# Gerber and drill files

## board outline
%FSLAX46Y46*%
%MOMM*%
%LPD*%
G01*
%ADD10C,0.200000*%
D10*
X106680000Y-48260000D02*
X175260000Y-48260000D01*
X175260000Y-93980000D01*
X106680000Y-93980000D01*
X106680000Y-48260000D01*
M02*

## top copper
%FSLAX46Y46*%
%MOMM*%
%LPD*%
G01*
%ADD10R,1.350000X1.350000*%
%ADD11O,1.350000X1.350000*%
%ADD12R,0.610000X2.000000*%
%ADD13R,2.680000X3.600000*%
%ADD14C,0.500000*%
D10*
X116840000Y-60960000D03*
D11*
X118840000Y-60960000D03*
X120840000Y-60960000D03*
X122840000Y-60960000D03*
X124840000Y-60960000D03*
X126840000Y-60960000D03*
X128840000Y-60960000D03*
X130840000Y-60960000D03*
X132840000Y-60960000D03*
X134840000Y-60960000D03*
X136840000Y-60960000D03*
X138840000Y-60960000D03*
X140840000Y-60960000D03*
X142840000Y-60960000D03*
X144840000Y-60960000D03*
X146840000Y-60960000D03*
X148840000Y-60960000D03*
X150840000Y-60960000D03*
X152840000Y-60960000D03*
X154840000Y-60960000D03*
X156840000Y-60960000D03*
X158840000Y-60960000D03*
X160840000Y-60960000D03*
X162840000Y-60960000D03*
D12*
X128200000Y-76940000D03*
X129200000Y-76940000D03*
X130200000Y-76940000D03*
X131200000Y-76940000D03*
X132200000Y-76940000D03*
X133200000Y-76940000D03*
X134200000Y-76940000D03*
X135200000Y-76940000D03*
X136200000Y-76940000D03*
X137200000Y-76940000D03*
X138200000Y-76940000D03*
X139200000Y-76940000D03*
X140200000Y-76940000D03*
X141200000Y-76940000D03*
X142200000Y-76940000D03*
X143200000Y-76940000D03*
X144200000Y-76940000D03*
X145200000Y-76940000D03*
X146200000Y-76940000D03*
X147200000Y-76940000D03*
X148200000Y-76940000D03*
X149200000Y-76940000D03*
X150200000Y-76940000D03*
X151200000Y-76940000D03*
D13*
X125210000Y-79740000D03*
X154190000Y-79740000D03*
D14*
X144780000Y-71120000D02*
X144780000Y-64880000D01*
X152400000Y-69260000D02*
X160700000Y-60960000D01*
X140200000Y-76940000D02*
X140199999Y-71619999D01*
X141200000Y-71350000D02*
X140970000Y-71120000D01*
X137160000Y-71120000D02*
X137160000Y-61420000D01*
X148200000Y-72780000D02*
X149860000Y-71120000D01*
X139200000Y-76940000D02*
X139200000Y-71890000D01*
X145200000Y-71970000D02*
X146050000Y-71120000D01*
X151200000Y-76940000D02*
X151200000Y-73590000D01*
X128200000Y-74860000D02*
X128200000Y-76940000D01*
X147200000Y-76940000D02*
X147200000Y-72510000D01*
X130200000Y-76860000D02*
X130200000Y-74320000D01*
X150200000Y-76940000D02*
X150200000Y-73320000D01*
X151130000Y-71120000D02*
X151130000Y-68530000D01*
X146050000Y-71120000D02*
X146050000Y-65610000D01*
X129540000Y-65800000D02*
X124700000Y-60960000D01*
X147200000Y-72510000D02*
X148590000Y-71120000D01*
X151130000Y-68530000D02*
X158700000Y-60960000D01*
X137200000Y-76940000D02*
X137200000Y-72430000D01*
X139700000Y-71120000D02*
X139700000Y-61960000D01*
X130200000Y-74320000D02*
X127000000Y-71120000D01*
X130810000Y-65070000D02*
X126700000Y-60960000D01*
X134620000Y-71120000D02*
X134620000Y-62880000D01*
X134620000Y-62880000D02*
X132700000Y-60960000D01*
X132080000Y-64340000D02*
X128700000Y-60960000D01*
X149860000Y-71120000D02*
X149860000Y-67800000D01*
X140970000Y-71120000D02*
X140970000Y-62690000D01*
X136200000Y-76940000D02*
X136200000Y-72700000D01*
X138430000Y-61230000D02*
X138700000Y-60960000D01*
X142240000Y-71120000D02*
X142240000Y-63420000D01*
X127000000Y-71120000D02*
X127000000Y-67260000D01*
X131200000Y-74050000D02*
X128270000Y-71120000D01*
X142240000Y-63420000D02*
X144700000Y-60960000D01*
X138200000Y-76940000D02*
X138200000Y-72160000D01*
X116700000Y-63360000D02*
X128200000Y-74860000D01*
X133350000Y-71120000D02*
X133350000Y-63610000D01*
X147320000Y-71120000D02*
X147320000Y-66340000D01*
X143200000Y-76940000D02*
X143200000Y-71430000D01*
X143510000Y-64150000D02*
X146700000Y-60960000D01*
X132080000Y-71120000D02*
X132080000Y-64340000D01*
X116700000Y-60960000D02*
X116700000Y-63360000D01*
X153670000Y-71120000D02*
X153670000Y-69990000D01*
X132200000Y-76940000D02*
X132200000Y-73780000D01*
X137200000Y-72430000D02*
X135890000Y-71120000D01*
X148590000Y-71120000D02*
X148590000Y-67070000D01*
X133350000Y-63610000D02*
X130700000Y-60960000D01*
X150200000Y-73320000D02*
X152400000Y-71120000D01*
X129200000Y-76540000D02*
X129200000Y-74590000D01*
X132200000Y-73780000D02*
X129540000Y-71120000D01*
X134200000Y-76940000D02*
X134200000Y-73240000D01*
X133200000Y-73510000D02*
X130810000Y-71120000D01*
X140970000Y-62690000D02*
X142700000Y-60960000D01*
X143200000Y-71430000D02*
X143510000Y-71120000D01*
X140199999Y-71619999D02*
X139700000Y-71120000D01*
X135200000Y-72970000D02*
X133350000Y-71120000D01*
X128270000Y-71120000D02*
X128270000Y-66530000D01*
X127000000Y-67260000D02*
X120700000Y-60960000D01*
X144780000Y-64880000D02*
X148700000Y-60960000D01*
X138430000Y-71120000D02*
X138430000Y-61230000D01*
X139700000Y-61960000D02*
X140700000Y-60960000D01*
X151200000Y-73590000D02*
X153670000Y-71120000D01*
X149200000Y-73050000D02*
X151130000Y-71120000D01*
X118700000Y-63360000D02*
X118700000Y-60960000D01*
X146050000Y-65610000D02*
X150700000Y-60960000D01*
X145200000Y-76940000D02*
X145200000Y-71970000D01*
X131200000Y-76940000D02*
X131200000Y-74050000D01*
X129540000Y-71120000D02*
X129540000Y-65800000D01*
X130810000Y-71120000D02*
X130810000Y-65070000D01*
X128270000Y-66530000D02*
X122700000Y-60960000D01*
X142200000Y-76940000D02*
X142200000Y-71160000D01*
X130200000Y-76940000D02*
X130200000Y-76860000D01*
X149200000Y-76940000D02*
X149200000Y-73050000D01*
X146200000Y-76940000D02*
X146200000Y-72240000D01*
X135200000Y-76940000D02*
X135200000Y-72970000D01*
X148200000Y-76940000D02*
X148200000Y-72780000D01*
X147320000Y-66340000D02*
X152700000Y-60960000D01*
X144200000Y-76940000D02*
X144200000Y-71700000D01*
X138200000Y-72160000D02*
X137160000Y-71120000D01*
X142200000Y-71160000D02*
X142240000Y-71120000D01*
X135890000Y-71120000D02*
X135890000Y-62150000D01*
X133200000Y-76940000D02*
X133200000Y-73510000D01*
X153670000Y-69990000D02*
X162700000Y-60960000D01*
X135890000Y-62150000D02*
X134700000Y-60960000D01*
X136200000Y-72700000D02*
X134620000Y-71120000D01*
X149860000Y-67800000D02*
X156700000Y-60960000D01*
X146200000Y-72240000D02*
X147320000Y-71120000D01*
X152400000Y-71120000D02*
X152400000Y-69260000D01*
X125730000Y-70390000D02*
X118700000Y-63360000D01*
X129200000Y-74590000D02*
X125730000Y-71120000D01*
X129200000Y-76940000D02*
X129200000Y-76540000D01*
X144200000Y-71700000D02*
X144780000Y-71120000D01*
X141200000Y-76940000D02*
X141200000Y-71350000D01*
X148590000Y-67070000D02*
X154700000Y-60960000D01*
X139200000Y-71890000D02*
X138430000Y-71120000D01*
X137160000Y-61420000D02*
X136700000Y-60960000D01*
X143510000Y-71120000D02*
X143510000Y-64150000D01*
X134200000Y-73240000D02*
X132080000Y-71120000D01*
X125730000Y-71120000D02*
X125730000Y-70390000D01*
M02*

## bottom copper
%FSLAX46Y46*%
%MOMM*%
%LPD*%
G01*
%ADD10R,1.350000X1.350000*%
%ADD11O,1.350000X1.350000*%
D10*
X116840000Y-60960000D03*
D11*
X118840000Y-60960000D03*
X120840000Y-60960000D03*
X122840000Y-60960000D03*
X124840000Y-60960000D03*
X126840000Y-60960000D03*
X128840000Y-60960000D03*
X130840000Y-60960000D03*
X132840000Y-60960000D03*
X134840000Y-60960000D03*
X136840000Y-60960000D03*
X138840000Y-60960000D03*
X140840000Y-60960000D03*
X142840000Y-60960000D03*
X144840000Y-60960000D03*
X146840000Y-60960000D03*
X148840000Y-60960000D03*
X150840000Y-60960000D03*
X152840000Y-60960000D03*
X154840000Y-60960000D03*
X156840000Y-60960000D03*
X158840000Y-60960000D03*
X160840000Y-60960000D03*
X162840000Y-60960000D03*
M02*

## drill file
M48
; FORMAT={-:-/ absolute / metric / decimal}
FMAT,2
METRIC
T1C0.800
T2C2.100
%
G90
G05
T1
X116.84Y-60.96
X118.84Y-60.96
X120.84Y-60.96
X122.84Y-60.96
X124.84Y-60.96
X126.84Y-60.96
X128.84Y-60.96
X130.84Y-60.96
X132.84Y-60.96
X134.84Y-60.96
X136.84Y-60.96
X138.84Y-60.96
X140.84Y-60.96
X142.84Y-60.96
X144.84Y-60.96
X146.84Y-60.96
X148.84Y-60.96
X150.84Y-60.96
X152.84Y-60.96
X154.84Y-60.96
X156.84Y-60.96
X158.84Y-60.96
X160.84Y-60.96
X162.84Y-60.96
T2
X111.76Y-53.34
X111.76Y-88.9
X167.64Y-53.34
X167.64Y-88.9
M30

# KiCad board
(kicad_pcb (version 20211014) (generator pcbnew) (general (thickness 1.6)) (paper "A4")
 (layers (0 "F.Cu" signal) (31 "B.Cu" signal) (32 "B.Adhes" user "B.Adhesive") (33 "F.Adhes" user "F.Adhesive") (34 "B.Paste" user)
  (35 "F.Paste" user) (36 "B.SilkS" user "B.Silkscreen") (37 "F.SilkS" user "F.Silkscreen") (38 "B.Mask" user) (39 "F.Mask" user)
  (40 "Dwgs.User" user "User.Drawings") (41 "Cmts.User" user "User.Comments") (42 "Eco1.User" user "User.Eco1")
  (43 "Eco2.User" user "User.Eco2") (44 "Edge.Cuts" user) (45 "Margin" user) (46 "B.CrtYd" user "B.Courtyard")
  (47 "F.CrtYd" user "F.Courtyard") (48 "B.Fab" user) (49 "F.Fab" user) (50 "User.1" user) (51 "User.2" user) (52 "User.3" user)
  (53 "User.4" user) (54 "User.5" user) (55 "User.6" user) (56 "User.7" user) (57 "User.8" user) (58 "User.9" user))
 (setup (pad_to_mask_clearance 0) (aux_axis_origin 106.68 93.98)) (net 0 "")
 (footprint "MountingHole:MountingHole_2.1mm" (layer "F.Cu") (at 111.76 53.34)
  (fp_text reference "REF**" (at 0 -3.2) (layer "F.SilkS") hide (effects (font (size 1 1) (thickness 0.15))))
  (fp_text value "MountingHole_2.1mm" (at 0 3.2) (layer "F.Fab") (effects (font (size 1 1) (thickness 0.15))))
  (pad "" np_thru_hole circle (at 0 0) (size 2.1 2.1) (drill 2.1) (layers *.Cu *.Mask)))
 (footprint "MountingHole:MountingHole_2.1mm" (layer "F.Cu") (at 167.64 53.34)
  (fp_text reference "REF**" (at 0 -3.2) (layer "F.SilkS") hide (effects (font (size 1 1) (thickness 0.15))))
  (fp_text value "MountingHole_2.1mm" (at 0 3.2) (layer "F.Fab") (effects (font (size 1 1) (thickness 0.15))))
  (pad "" np_thru_hole circle (at 0 0) (size 2.1 2.1) (drill 2.1) (layers *.Cu *.Mask)))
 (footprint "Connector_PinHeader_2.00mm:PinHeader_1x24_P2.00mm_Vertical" (layer "F.Cu") (at 116.84 60.96 90)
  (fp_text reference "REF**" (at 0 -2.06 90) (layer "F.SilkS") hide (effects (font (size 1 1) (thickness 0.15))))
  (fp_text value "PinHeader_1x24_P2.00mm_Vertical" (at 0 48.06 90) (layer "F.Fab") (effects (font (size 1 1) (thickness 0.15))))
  (pad "1" thru_hole rect (at 0 0 90) (size 1.35 1.35) (drill 0.8) (layers *.Cu *.Mask))
  (pad "2" thru_hole oval (at 0 2 90) (size 1.35 1.35) (drill 0.8) (layers *.Cu *.Mask))
  (pad "3" thru_hole oval (at 0 4 90) (size 1.35 1.35) (drill 0.8) (layers *.Cu *.Mask))
  (pad "4" thru_hole oval (at 0 6 90) (size 1.35 1.35) (drill 0.8) (layers *.Cu *.Mask))
  (pad "5" thru_hole oval (at 0 8 90) (size 1.35 1.35) (drill 0.8) (layers *.Cu *.Mask))
  (pad "6" thru_hole oval (at 0 10 90) (size 1.35 1.35) (drill 0.8) (layers *.Cu *.Mask))
  (pad "7" thru_hole oval (at 0 12 90) (size 1.35 1.35) (drill 0.8) (layers *.Cu *.Mask))
  (pad "8" thru_hole oval (at 0 14 90) (size 1.35 1.35) (drill 0.8) (layers *.Cu *.Mask))
  (pad "9" thru_hole oval (at 0 16 90) (size 1.35 1.35) (drill 0.8) (layers *.Cu *.Mask))
  (pad "10" thru_hole oval (at 0 18 90) (size 1.35 1.35) (drill 0.8) (layers *.Cu *.Mask))
  (pad "11" thru_hole oval (at 0 20 90) (size 1.35 1.35) (drill 0.8) (layers *.Cu *.Mask))
  (pad "12" thru_hole oval (at 0 22 90) (size 1.35 1.35) (drill 0.8) (layers *.Cu *.Mask))
  (pad "13" thru_hole oval (at 0 24 90) (size 1.35 1.35) (drill 0.8) (layers *.Cu *.Mask))
  (pad "14" thru_hole oval (at 0 26 90) (size 1.35 1.35) (drill 0.8) (layers *.Cu *.Mask))
  (pad "15" thru_hole oval (at 0 28 90) (size 1.35 1.35) (drill 0.8) (layers *.Cu *.Mask))
  (pad "16" thru_hole oval (at 0 30 90) (size 1.35 1.35) (drill 0.8) (layers *.Cu *.Mask))
  (pad "17" thru_hole oval (at 0 32 90) (size 1.35 1.35) (drill 0.8) (layers *.Cu *.Mask))
  (pad "18" thru_hole oval (at 0 34 90) (size 1.35 1.35) (drill 0.8) (layers *.Cu *.Mask))
  (pad "19" thru_hole oval (at 0 36 90) (size 1.35 1.35) (drill 0.8) (layers *.Cu *.Mask))
  (pad "20" thru_hole oval (at 0 38 90) (size 1.35 1.35) (drill 0.8) (layers *.Cu *.Mask))
  (pad "21" thru_hole oval (at 0 40 90) (size 1.35 1.35) (drill 0.8) (layers *.Cu *.Mask))
  (pad "22" thru_hole oval (at 0 42 90) (size 1.35 1.35) (drill 0.8) (layers *.Cu *.Mask))
  (pad "23" thru_hole oval (at 0 44 90) (size 1.35 1.35) (drill 0.8) (layers *.Cu *.Mask))
  (pad "24" thru_hole oval (at 0 46 90) (size 1.35 1.35) (drill 0.8) (layers *.Cu *.Mask)))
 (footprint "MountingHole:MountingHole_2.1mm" (layer "F.Cu") (at 111.76 88.9)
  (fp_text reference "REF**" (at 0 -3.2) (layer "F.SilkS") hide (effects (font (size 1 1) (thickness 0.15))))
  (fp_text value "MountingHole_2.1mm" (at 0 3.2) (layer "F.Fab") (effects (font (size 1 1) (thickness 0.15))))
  (pad "" np_thru_hole circle (at 0 0) (size 2.1 2.1) (drill 2.1) (layers *.Cu *.Mask)))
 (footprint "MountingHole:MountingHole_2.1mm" (layer "F.Cu") (at 167.64 88.9)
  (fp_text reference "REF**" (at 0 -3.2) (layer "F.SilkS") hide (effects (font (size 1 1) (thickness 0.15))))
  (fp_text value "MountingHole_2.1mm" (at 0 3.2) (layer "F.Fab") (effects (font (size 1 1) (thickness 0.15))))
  (pad "" np_thru_hole circle (at 0 0) (size 2.1 2.1) (drill 2.1) (layers *.Cu *.Mask)))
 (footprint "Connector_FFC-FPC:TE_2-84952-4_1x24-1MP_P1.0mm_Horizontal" (layer "F.Cu") (at 139.7 78.74)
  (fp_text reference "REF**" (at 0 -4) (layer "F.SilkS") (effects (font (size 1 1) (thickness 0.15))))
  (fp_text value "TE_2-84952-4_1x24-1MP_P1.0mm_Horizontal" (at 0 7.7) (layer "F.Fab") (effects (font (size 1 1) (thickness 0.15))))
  (pad "1" smd rect (at -11.5 -1.8) (size 0.61 2) (layers "F.Cu" "F.Paste" "F.Mask"))
  (pad "2" smd rect (at -10.5 -1.8) (size 0.61 2) (layers "F.Cu" "F.Paste" "F.Mask"))
  (pad "3" smd rect (at -9.5 -1.8) (size 0.61 2) (layers "F.Cu" "F.Paste" "F.Mask"))
  (pad "4" smd rect (at -8.5 -1.8) (size 0.61 2) (layers "F.Cu" "F.Paste" "F.Mask"))
  (pad "5" smd rect (at -7.5 -1.8) (size 0.61 2) (layers "F.Cu" "F.Paste" "F.Mask"))
  (pad "6" smd rect (at -6.5 -1.8) (size 0.61 2) (layers "F.Cu" "F.Paste" "F.Mask"))
  (pad "7" smd rect (at -5.5 -1.8) (size 0.61 2) (layers "F.Cu" "F.Paste" "F.Mask"))
  (pad "8" smd rect (at -4.5 -1.8) (size 0.61 2) (layers "F.Cu" "F.Paste" "F.Mask"))
  (pad "9" smd rect (at -3.5 -1.8) (size 0.61 2) (layers "F.Cu" "F.Paste" "F.Mask"))
  (pad "10" smd rect (at -2.5 -1.8) (size 0.61 2) (layers "F.Cu" "F.Paste" "F.Mask"))
  (pad "11" smd rect (at -1.5 -1.8) (size 0.61 2) (layers "F.Cu" "F.Paste" "F.Mask"))
  (pad "12" smd rect (at -0.5 -1.8) (size 0.61 2) (layers "F.Cu" "F.Paste" "F.Mask"))
  (pad "13" smd rect (at 0.5 -1.8) (size 0.61 2) (layers "F.Cu" "F.Paste" "F.Mask"))
  (pad "14" smd rect (at 1.5 -1.8) (size 0.61 2) (layers "F.Cu" "F.Paste" "F.Mask"))
  (pad "15" smd rect (at 2.5 -1.8) (size 0.61 2) (layers "F.Cu" "F.Paste" "F.Mask"))
  (pad "16" smd rect (at 3.5 -1.8) (size 0.61 2) (layers "F.Cu" "F.Paste" "F.Mask"))
  (pad "17" smd rect (at 4.5 -1.8) (size 0.61 2) (layers "F.Cu" "F.Paste" "F.Mask"))
  (pad "18" smd rect (at 5.5 -1.8) (size 0.61 2) (layers "F.Cu" "F.Paste" "F.Mask"))
  (pad "19" smd rect (at 6.5 -1.8) (size 0.61 2) (layers "F.Cu" "F.Paste" "F.Mask"))
  (pad "20" smd rect (at 7.5 -1.8) (size 0.61 2) (layers "F.Cu" "F.Paste" "F.Mask"))
  (pad "21" smd rect (at 8.5 -1.8) (size 0.61 2) (layers "F.Cu" "F.Paste" "F.Mask"))
  (pad "22" smd rect (at 9.5 -1.8) (size 0.61 2) (layers "F.Cu" "F.Paste" "F.Mask"))
  (pad "23" smd rect (at 10.5 -1.8) (size 0.61 2) (layers "F.Cu" "F.Paste" "F.Mask"))
  (pad "24" smd rect (at 11.5 -1.8) (size 0.61 2) (layers "F.Cu" "F.Paste" "F.Mask"))
  (pad "MP" smd rect (at -14.49 1) (size 2.68 3.6) (layers "F.Cu" "F.Paste" "F.Mask"))
  (pad "MP" smd rect (at 14.49 1) (size 2.68 3.6) (layers "F.Cu" "F.Paste" "F.Mask")))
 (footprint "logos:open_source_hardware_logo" (layer "F.Cu") (at 167.64 71.12)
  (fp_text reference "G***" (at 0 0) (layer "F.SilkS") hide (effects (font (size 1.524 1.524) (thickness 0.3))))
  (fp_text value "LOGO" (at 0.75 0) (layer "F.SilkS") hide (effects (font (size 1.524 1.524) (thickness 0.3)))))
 (gr_rect (start 175.26 48.26) (end 106.68 93.98) (layer "Edge.Cuts") (width 0.2) (fill none))
 (segment (start 144.78 71.12) (end 144.78 64.88) (width 0.5) (layer "F.Cu") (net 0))
 (segment (start 152.4 69.26) (end 160.7 60.96) (width 0.5) (layer "F.Cu") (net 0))
 (segment (start 140.2 76.94) (end 140.199999 71.619999) (width 0.5) (layer "F.Cu") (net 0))
 (segment (start 141.2 71.35) (end 140.97 71.12) (width 0.5) (layer "F.Cu") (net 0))
 (segment (start 137.16 71.12) (end 137.16 61.42) (width 0.5) (layer "F.Cu") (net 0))
 (segment (start 148.2 72.78) (end 149.86 71.12) (width 0.5) (layer "F.Cu") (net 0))
 (segment (start 139.2 76.94) (end 139.2 71.89) (width 0.5) (layer "F.Cu") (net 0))
 (segment (start 145.2 71.97) (end 146.05 71.12) (width 0.5) (layer "F.Cu") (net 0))
 (segment (start 151.2 76.94) (end 151.2 73.59) (width 0.5) (layer "F.Cu") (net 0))
 (segment (start 128.2 74.86) (end 128.2 76.94) (width 0.5) (layer "F.Cu") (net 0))
 (segment (start 147.2 76.94) (end 147.2 72.51) (width 0.5) (layer "F.Cu") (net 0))
 (segment (start 130.2 76.86) (end 130.2 74.32) (width 0.5) (layer "F.Cu") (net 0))
 (segment (start 150.2 76.94) (end 150.2 73.32) (width 0.5) (layer "F.Cu") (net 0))
 (segment (start 151.13 71.12) (end 151.13 68.53) (width 0.5) (layer "F.Cu") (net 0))
 (segment (start 146.05 71.12) (end 146.05 65.61) (width 0.5) (layer "F.Cu") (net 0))
 (segment (start 129.54 65.8) (end 124.7 60.96) (width 0.5) (layer "F.Cu") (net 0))
 (segment (start 147.2 72.51) (end 148.59 71.12) (width 0.5) (layer "F.Cu") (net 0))
 (segment (start 151.13 68.53) (end 158.7 60.96) (width 0.5) (layer "F.Cu") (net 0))
 (segment (start 137.2 76.94) (end 137.2 72.43) (width 0.5) (layer "F.Cu") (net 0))
 (segment (start 139.7 71.12) (end 139.7 61.96) (width 0.5) (layer "F.Cu") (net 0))
 (segment (start 130.2 74.32) (end 127 71.12) (width 0.5) (layer "F.Cu") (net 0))
 (segment (start 130.81 65.07) (end 126.7 60.96) (width 0.5) (layer "F.Cu") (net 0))
 (segment (start 134.62 71.12) (end 134.62 62.88) (width 0.5) (layer "F.Cu") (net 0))
 (segment (start 134.62 62.88) (end 132.7 60.96) (width 0.5) (layer "F.Cu") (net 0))
 (segment (start 132.08 64.34) (end 128.7 60.96) (width 0.5) (layer "F.Cu") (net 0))
 (segment (start 149.86 71.12) (end 149.86 67.8) (width 0.5) (layer "F.Cu") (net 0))
 (segment (start 140.97 71.12) (end 140.97 62.69) (width 0.5) (layer "F.Cu") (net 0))
 (segment (start 136.2 76.94) (end 136.2 72.7) (width 0.5) (layer "F.Cu") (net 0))
 (segment (start 138.43 61.23) (end 138.7 60.96) (width 0.5) (layer "F.Cu") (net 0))
 (segment (start 142.24 71.12) (end 142.24 63.42) (width 0.5) (layer "F.Cu") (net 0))
 (segment (start 127 71.12) (end 127 67.26) (width 0.5) (layer "F.Cu") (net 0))
 (segment (start 131.2 74.05) (end 128.27 71.12) (width 0.5) (layer "F.Cu") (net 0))
 (segment (start 142.24 63.42) (end 144.7 60.96) (width 0.5) (layer "F.Cu") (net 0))
 (segment (start 138.2 76.94) (end 138.2 72.16) (width 0.5) (layer "F.Cu") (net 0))
 (segment (start 116.7 63.36) (end 128.2 74.86) (width 0.5) (layer "F.Cu") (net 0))
 (segment (start 133.35 71.12) (end 133.35 63.61) (width 0.5) (layer "F.Cu") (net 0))
 (segment (start 147.32 71.12) (end 147.32 66.34) (width 0.5) (layer "F.Cu") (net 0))
 (segment (start 143.2 76.94) (end 143.2 71.43) (width 0.5) (layer "F.Cu") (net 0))
 (segment (start 143.51 64.15) (end 146.7 60.96) (width 0.5) (layer "F.Cu") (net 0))
 (segment (start 132.08 71.12) (end 132.08 64.34) (width 0.5) (layer "F.Cu") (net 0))
 (segment (start 116.7 60.96) (end 116.7 63.36) (width 0.5) (layer "F.Cu") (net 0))
 (segment (start 153.67 71.12) (end 153.67 69.99) (width 0.5) (layer "F.Cu") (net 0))
 (segment (start 132.2 76.94) (end 132.2 73.78) (width 0.5) (layer "F.Cu") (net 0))
 (segment (start 137.2 72.43) (end 135.89 71.12) (width 0.5) (layer "F.Cu") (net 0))
 (segment (start 148.59 71.12) (end 148.59 67.07) (width 0.5) (layer "F.Cu") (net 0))
 (segment (start 133.35 63.61) (end 130.7 60.96) (width 0.5) (layer "F.Cu") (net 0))
 (segment (start 150.2 73.32) (end 152.4 71.12) (width 0.5) (layer "F.Cu") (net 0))
 (segment (start 129.2 76.54) (end 129.2 74.59) (width 0.5) (layer "F.Cu") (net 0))
 (segment (start 132.2 73.78) (end 129.54 71.12) (width 0.5) (layer "F.Cu") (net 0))
 (segment (start 134.2 76.94) (end 134.2 73.24) (width 0.5) (layer "F.Cu") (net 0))
 (segment (start 133.2 73.51) (end 130.81 71.12) (width 0.5) (layer "F.Cu") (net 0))
 (segment (start 140.97 62.69) (end 142.7 60.96) (width 0.5) (layer "F.Cu") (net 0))
 (segment (start 143.2 71.43) (end 143.51 71.12) (width 0.5) (layer "F.Cu") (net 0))
 (segment (start 140.199999 71.619999) (end 139.7 71.12) (width 0.5) (layer "F.Cu") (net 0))
 (segment (start 135.2 72.97) (end 133.35 71.12) (width 0.5) (layer "F.Cu") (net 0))
 (segment (start 128.27 71.12) (end 128.27 66.53) (width 0.5) (layer "F.Cu") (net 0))
 (segment (start 127 67.26) (end 120.7 60.96) (width 0.5) (layer "F.Cu") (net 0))
 (segment (start 144.78 64.88) (end 148.7 60.96) (width 0.5) (layer "F.Cu") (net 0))
 (segment (start 138.43 71.12) (end 138.43 61.23) (width 0.5) (layer "F.Cu") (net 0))
 (segment (start 139.7 61.96) (end 140.7 60.96) (width 0.5) (layer "F.Cu") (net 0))
 (segment (start 151.2 73.59) (end 153.67 71.12) (width 0.5) (layer "F.Cu") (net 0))
 (segment (start 149.2 73.05) (end 151.13 71.12) (width 0.5) (layer "F.Cu") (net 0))
 (segment (start 118.7 63.36) (end 118.7 60.96) (width 0.5) (layer "F.Cu") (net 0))
 (segment (start 146.05 65.61) (end 150.7 60.96) (width 0.5) (layer "F.Cu") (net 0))
 (segment (start 145.2 76.94) (end 145.2 71.97) (width 0.5) (layer "F.Cu") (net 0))
 (segment (start 131.2 76.94) (end 131.2 74.05) (width 0.5) (layer "F.Cu") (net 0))
 (segment (start 129.54 71.12) (end 129.54 65.8) (width 0.5) (layer "F.Cu") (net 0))
 (segment (start 130.81 71.12) (end 130.81 65.07) (width 0.5) (layer "F.Cu") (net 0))
 (segment (start 128.27 66.53) (end 122.7 60.96) (width 0.5) (layer "F.Cu") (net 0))
 (segment (start 142.2 76.94) (end 142.2 71.16) (width 0.5) (layer "F.Cu") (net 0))
 (segment (start 130.2 76.94) (end 130.2 76.86) (width 0.5) (layer "F.Cu") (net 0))
 (segment (start 149.2 76.94) (end 149.2 73.05) (width 0.5) (layer "F.Cu") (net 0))
 (segment (start 146.2 76.94) (end 146.2 72.24) (width 0.5) (layer "F.Cu") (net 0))
 (segment (start 135.2 76.94) (end 135.2 72.97) (width 0.5) (layer "F.Cu") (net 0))
 (segment (start 148.2 76.94) (end 148.2 72.78) (width 0.5) (layer "F.Cu") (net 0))
 (segment (start 147.32 66.34) (end 152.7 60.96) (width 0.5) (layer "F.Cu") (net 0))
 (segment (start 144.2 76.94) (end 144.2 71.7) (width 0.5) (layer "F.Cu") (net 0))
 (segment (start 138.2 72.16) (end 137.16 71.12) (width 0.5) (layer "F.Cu") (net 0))
 (segment (start 142.2 71.16) (end 142.24 71.12) (width 0.5) (layer "F.Cu") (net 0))
 (segment (start 135.89 71.12) (end 135.89 62.15) (width 0.5) (layer "F.Cu") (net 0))
 (segment (start 133.2 76.94) (end 133.2 73.51) (width 0.5) (layer "F.Cu") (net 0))
 (segment (start 153.67 69.99) (end 162.7 60.96) (width 0.5) (layer "F.Cu") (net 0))
 (segment (start 135.89 62.15) (end 134.7 60.96) (width 0.5) (layer "F.Cu") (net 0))
 (segment (start 136.2 72.7) (end 134.62 71.12) (width 0.5) (layer "F.Cu") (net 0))
 (segment (start 149.86 67.8) (end 156.7 60.96) (width 0.5) (layer "F.Cu") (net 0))
 (segment (start 146.2 72.24) (end 147.32 71.12) (width 0.5) (layer "F.Cu") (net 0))
 (segment (start 152.4 71.12) (end 152.4 69.26) (width 0.5) (layer "F.Cu") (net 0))
 (segment (start 125.73 70.39) (end 118.7 63.36) (width 0.5) (layer "F.Cu") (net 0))
 (segment (start 129.2 74.59) (end 125.73 71.12) (width 0.5) (layer "F.Cu") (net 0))
 (segment (start 129.2 76.94) (end 129.2 76.54) (width 0.5) (layer "F.Cu") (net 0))
 (segment (start 144.2 71.7) (end 144.78 71.12) (width 0.5) (layer "F.Cu") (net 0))
 (segment (start 141.2 76.94) (end 141.2 71.35) (width 0.5) (layer "F.Cu") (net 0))
 (segment (start 148.59 67.07) (end 154.7 60.96) (width 0.5) (layer "F.Cu") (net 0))
 (segment (start 139.2 71.89) (end 138.43 71.12) (width 0.5) (layer "F.Cu") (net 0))
 (segment (start 137.16 61.42) (end 136.7 60.96) (width 0.5) (layer "F.Cu") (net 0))
 (segment (start 143.51 71.12) (end 143.51 64.15) (width 0.5) (layer "F.Cu") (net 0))
 (segment (start 134.2 73.24) (end 132.08 71.12) (width 0.5) (layer "F.Cu") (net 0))
 (segment (start 125.73 71.12) (end 125.73 70.39) (width 0.5) (layer "F.Cu") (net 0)))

